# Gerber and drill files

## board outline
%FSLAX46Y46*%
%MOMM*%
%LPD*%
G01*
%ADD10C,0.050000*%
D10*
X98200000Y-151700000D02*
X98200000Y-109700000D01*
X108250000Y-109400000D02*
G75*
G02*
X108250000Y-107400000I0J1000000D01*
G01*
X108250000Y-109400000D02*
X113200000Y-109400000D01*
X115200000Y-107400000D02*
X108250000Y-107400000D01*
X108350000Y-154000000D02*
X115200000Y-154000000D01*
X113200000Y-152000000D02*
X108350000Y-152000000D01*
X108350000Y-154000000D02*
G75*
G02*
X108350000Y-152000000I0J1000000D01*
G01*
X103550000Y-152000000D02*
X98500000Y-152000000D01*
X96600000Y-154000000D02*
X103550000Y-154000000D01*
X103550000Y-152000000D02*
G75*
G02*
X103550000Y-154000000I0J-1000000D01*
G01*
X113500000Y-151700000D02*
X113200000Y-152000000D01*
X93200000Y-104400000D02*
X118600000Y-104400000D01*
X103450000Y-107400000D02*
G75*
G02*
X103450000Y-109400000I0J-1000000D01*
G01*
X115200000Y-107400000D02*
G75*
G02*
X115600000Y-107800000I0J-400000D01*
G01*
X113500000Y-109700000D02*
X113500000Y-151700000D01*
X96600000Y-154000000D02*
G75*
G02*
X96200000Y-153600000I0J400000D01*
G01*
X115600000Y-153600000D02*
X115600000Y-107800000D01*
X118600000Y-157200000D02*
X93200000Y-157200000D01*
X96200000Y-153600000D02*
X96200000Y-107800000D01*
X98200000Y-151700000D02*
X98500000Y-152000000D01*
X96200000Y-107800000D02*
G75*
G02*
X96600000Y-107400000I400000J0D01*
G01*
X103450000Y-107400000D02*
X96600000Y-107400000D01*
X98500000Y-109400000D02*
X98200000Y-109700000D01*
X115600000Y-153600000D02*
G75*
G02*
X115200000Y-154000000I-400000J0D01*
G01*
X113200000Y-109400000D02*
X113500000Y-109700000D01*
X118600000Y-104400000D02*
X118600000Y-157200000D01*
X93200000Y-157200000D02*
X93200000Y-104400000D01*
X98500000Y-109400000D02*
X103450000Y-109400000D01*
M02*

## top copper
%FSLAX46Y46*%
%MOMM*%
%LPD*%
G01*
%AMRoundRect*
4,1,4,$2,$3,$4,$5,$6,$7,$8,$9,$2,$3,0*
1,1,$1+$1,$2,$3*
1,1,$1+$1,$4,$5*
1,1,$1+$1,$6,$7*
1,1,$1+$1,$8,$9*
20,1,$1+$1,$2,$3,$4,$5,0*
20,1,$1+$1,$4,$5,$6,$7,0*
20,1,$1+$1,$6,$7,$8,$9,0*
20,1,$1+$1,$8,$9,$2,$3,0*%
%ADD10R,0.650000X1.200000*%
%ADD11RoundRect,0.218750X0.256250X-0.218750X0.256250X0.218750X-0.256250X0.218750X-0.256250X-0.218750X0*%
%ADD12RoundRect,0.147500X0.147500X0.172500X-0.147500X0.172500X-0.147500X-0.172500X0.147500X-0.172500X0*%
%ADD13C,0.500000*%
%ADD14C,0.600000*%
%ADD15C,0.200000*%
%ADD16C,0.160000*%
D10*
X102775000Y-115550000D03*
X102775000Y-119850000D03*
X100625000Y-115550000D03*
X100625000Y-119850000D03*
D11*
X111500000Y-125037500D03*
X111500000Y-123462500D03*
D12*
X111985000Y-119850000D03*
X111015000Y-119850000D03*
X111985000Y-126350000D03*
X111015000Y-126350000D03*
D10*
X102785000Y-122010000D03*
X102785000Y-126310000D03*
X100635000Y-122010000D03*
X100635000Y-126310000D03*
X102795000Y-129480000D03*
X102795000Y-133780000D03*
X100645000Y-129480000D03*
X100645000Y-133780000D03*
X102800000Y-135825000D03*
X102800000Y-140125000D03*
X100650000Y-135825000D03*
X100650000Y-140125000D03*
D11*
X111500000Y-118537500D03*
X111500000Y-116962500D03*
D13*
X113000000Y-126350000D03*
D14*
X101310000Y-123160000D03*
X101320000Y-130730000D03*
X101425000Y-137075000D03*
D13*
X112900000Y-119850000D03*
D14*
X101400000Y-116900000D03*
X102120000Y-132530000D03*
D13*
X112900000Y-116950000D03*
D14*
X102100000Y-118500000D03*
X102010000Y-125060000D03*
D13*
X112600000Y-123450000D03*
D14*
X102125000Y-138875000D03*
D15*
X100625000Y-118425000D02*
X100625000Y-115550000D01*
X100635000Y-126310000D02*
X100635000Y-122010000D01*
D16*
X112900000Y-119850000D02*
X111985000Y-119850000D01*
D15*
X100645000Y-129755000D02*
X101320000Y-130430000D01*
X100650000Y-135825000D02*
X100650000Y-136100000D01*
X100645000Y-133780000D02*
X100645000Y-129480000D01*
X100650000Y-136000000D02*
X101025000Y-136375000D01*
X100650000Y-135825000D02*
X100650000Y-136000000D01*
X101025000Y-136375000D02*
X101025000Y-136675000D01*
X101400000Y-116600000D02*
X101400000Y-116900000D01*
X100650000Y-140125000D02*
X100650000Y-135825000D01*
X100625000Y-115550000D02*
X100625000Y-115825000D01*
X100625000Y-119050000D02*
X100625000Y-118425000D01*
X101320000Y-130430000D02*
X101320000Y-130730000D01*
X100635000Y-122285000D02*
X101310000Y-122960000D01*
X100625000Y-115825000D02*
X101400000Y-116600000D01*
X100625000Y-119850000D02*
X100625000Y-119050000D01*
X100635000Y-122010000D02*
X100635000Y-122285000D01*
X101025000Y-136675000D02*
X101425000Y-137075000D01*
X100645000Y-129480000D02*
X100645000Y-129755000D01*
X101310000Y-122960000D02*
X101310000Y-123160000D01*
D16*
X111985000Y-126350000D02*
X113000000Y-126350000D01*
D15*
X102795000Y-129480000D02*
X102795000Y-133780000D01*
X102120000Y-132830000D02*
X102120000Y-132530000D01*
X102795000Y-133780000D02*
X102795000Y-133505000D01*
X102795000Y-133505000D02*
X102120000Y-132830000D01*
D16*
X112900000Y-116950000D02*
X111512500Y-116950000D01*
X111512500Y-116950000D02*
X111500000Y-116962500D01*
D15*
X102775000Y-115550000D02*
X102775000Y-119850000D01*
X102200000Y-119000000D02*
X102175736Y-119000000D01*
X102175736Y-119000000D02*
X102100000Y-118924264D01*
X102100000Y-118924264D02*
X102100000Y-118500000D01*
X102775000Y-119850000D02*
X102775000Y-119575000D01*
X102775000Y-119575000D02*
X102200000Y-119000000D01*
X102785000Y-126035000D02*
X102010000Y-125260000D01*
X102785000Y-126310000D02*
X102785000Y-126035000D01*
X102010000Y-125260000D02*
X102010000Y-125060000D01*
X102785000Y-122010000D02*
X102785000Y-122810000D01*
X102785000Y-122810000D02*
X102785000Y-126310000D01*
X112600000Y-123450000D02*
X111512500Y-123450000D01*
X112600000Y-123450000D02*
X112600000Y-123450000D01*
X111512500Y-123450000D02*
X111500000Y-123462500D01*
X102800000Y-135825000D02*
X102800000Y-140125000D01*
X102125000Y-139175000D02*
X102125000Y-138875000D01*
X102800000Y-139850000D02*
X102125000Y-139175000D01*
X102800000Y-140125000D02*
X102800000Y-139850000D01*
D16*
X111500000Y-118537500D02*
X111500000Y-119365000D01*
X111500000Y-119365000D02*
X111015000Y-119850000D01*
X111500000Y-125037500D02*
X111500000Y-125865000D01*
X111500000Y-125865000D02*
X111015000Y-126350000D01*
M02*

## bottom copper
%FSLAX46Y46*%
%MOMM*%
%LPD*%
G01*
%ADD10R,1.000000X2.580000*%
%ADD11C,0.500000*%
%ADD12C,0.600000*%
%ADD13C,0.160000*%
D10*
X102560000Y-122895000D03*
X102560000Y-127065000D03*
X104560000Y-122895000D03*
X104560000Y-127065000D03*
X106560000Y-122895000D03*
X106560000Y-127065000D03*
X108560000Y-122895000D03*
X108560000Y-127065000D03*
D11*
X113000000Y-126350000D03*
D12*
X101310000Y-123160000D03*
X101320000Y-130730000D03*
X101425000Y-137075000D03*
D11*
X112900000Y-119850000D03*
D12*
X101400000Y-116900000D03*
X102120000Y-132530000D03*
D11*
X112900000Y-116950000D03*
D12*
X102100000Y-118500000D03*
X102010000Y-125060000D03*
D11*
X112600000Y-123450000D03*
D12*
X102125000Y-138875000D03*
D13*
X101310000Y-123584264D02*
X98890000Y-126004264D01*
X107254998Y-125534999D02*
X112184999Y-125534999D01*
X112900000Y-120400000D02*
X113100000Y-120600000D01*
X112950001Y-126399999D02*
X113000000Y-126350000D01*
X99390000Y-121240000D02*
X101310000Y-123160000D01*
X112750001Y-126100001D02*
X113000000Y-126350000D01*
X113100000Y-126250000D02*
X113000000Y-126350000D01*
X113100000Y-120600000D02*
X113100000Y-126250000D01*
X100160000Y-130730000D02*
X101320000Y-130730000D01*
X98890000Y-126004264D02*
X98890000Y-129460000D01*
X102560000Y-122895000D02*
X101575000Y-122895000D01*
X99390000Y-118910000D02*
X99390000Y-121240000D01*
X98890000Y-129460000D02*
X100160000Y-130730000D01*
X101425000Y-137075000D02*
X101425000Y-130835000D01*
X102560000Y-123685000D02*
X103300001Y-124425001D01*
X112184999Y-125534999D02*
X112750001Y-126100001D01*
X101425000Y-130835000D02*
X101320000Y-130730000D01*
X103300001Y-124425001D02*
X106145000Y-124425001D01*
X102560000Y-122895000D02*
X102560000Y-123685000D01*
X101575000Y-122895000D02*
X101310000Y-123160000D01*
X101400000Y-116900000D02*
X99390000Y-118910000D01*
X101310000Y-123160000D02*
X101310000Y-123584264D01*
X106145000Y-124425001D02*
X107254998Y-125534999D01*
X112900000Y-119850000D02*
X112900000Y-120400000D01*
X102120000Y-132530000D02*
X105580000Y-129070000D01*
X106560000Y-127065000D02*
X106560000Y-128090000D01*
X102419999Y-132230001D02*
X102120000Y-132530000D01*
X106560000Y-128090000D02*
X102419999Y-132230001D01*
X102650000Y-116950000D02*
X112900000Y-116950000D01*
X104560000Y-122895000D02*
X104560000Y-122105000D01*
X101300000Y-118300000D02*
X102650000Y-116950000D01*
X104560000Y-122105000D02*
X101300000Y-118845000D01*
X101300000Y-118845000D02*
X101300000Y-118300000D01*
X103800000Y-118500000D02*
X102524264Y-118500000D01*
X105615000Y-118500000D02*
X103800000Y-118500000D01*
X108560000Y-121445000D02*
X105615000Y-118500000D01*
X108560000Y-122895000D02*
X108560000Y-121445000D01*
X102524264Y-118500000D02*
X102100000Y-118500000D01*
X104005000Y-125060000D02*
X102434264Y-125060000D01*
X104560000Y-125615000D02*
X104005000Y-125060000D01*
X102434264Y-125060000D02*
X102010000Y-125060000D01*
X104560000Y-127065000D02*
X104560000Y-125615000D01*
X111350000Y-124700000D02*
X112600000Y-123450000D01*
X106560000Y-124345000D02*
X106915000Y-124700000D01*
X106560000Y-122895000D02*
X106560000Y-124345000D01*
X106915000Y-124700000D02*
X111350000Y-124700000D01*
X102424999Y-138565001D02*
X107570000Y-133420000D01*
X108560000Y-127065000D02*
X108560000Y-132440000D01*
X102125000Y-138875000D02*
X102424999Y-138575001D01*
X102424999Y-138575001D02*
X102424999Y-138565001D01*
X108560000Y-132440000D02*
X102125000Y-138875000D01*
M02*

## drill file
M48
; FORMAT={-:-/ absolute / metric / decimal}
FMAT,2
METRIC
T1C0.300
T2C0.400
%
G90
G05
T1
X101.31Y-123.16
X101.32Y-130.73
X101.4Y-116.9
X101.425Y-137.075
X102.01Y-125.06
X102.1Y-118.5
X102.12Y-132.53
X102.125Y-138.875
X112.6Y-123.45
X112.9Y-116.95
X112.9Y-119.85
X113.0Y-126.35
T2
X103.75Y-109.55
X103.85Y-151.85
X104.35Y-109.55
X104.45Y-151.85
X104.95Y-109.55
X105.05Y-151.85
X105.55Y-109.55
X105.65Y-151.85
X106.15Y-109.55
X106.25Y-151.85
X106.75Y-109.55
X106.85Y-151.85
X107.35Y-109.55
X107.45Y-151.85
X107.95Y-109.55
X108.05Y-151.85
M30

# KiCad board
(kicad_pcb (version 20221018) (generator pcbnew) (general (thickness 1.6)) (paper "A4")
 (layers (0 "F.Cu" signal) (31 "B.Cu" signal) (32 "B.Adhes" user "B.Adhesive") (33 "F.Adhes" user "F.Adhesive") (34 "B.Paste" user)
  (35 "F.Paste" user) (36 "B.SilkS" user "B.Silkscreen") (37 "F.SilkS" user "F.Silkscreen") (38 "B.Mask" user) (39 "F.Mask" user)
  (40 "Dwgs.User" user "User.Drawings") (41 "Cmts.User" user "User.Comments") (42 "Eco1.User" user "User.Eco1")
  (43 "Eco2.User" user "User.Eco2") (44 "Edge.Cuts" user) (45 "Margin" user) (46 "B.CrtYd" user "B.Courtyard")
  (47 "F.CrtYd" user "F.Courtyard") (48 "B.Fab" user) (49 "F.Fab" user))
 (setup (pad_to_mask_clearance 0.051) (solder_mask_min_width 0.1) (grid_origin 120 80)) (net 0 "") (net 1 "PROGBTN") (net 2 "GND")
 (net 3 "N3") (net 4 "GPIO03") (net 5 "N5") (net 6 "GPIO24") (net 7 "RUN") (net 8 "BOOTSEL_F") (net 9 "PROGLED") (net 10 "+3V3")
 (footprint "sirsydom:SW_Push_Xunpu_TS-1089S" (layer "F.Cu") (at 101.7 117.7 -90)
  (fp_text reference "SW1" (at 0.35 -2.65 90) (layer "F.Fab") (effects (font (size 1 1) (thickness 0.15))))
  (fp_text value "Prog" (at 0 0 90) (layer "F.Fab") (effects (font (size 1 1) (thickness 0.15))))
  (pad "1" smd rect (at -2.15 -1.075 270) (size 1.2 0.65) (layers "F.Cu" "F.Paste" "F.Mask") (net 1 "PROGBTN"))
  (pad "1" smd rect (at 2.15 -1.075 270) (size 1.2 0.65) (layers "F.Cu" "F.Paste" "F.Mask") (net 1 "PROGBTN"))
  (pad "2" smd rect (at -2.15 1.075 270) (size 1.2 0.65) (layers "F.Cu" "F.Paste" "F.Mask") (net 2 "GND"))
  (pad "2" smd rect (at 2.15 1.075 270) (size 1.2 0.65) (layers "F.Cu" "F.Paste" "F.Mask") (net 2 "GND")))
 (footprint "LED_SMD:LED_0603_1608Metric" (layer "F.Cu") (at 111.5 124.25 90)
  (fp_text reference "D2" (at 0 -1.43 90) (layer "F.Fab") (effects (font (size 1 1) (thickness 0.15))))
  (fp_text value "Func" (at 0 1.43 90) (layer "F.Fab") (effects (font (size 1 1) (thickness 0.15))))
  (pad "1" smd roundrect (at -0.7875 0 90) (size 0.875 0.95) (layers "F.Cu" "F.Paste" "F.Mask") (roundrect_rratio 0.25) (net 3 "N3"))
  (pad "2" smd roundrect (at 0.7875 0 90) (size 0.875 0.95) (layers "F.Cu" "F.Paste" "F.Mask") (roundrect_rratio 0.25) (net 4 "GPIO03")))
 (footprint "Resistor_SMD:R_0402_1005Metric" (layer "F.Cu") (at 111.5 119.85 180)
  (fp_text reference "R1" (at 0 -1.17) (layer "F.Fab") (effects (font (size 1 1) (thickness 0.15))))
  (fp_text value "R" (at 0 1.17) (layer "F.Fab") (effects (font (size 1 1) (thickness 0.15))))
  (pad "1" smd roundrect (at -0.485 0 180) (size 0.59 0.64) (layers "F.Cu" "F.Paste" "F.Mask") (roundrect_rratio 0.25) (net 2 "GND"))
  (pad "2" smd roundrect (at 0.485 0 180) (size 0.59 0.64) (layers "F.Cu" "F.Paste" "F.Mask") (roundrect_rratio 0.25) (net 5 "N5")))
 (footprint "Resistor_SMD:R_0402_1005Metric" (layer "F.Cu") (at 111.5 126.35 180)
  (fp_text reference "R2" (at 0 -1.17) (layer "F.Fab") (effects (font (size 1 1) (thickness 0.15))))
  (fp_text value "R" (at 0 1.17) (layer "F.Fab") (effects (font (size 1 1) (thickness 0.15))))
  (pad "1" smd roundrect (at -0.485 0 180) (size 0.59 0.64) (layers "F.Cu" "F.Paste" "F.Mask") (roundrect_rratio 0.25) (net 2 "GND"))
  (pad "2" smd roundrect (at 0.485 0 180) (size 0.59 0.64) (layers "F.Cu" "F.Paste" "F.Mask") (roundrect_rratio 0.25) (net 3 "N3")))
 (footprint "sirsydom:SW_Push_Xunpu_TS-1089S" (layer "F.Cu") (at 101.71 124.16 -90)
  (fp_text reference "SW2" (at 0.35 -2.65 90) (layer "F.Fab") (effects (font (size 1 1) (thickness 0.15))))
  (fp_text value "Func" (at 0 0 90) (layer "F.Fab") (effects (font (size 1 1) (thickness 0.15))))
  (pad "1" smd rect (at -2.15 -1.075 270) (size 1.2 0.65) (layers "F.Cu" "F.Paste" "F.Mask") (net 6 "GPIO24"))
  (pad "1" smd rect (at 2.15 -1.075 270) (size 1.2 0.65) (layers "F.Cu" "F.Paste" "F.Mask") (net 6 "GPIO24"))
  (pad "2" smd rect (at -2.15 1.075 270) (size 1.2 0.65) (layers "F.Cu" "F.Paste" "F.Mask") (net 2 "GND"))
  (pad "2" smd rect (at 2.15 1.075 270) (size 1.2 0.65) (layers "F.Cu" "F.Paste" "F.Mask") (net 2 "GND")))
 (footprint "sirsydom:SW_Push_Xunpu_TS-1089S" (layer "F.Cu") (at 101.72 131.63 -90)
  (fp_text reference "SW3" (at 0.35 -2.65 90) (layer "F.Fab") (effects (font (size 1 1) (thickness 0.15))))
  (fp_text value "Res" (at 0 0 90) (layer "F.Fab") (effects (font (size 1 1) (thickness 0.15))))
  (pad "1" smd rect (at -2.15 -1.075 270) (size 1.2 0.65) (layers "F.Cu" "F.Paste" "F.Mask") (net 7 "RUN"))
  (pad "1" smd rect (at 2.15 -1.075 270) (size 1.2 0.65) (layers "F.Cu" "F.Paste" "F.Mask") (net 7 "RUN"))
  (pad "2" smd rect (at -2.15 1.075 270) (size 1.2 0.65) (layers "F.Cu" "F.Paste" "F.Mask") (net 2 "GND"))
  (pad "2" smd rect (at 2.15 1.075 270) (size 1.2 0.65) (layers "F.Cu" "F.Paste" "F.Mask") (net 2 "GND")))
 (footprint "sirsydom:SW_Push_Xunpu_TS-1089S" (layer "F.Cu") (at 101.725 137.975 -90)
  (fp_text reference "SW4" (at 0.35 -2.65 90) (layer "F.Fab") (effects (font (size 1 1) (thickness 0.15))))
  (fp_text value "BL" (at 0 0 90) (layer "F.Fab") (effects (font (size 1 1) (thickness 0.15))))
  (pad "1" smd rect (at -2.15 -1.075 270) (size 1.2 0.65) (layers "F.Cu" "F.Paste" "F.Mask") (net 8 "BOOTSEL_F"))
  (pad "1" smd rect (at 2.15 -1.075 270) (size 1.2 0.65) (layers "F.Cu" "F.Paste" "F.Mask") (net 8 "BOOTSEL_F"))
  (pad "2" smd rect (at -2.15 1.075 270) (size 1.2 0.65) (layers "F.Cu" "F.Paste" "F.Mask") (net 2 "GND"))
  (pad "2" smd rect (at 2.15 1.075 270) (size 1.2 0.65) (layers "F.Cu" "F.Paste" "F.Mask") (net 2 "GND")))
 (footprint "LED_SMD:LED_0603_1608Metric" (layer "F.Cu") (at 111.5 117.75 90)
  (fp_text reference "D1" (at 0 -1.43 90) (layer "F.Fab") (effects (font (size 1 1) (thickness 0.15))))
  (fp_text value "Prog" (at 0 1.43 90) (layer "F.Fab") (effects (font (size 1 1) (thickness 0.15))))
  (pad "1" smd roundrect (at -0.7875 0 90) (size 0.875 0.95) (layers "F.Cu" "F.Paste" "F.Mask") (roundrect_rratio 0.25) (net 5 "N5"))
  (pad "2" smd roundrect (at 0.7875 0 90) (size 0.875 0.95) (layers "F.Cu" "F.Paste" "F.Mask") (roundrect_rratio 0.25) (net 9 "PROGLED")))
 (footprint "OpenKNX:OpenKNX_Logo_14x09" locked (layer "F.Cu") (at 105.8 146.4)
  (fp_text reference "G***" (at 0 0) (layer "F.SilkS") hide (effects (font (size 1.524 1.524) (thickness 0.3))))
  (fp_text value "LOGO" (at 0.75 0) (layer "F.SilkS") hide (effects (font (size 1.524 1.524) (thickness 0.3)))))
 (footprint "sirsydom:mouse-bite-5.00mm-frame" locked (layer "F.Cu") (at 105.35 109.55)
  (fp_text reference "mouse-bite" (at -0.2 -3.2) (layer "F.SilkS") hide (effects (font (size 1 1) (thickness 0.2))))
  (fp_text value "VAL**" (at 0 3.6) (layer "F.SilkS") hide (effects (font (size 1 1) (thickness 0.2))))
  (pad "" np_thru_hole circle locked (at -1.6 0) (size 0.4 0.4) (drill 0.4) (layers "*.Cu" "*.Mask"))
  (pad "" np_thru_hole circle locked (at -1 0) (size 0.4 0.4) (drill 0.4) (layers "*.Cu" "*.Mask"))
  (pad "" np_thru_hole circle locked (at -0.4 0) (size 0.4 0.4) (drill 0.4) (layers "*.Cu" "*.Mask"))
  (pad "" np_thru_hole circle locked (at 0.2 0) (size 0.4 0.4) (drill 0.4) (layers "*.Cu" "*.Mask"))
  (pad "" np_thru_hole circle locked (at 0.8 0) (size 0.4 0.4) (drill 0.4) (layers "*.Cu" "*.Mask"))
  (pad "" np_thru_hole circle locked (at 1.4 0) (size 0.4 0.4) (drill 0.4) (layers "*.Cu" "*.Mask"))
  (pad "" np_thru_hole circle locked (at 2 0) (size 0.4 0.4) (drill 0.4) (layers "*.Cu" "*.Mask"))
  (pad "" np_thru_hole circle locked (at 2.6 0) (size 0.4 0.4) (drill 0.4) (layers "*.Cu" "*.Mask")))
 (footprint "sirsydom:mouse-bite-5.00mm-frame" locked (layer "F.Cu") (at 106.45 151.85 180)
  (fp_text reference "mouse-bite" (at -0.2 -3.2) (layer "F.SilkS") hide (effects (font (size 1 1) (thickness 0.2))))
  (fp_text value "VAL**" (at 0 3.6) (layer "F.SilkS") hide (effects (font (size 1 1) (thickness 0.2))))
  (pad "" np_thru_hole circle locked (at -1.6 0 180) (size 0.4 0.4) (drill 0.4) (layers "*.Cu" "*.Mask"))
  (pad "" np_thru_hole circle locked (at -1 0 180) (size 0.4 0.4) (drill 0.4) (layers "*.Cu" "*.Mask"))
  (pad "" np_thru_hole circle locked (at -0.4 0 180) (size 0.4 0.4) (drill 0.4) (layers "*.Cu" "*.Mask"))
  (pad "" np_thru_hole circle locked (at 0.2 0 180) (size 0.4 0.4) (drill 0.4) (layers "*.Cu" "*.Mask"))
  (pad "" np_thru_hole circle locked (at 0.8 0 180) (size 0.4 0.4) (drill 0.4) (layers "*.Cu" "*.Mask"))
  (pad "" np_thru_hole circle locked (at 1.4 0 180) (size 0.4 0.4) (drill 0.4) (layers "*.Cu" "*.Mask"))
  (pad "" np_thru_hole circle locked (at 2 0 180) (size 0.4 0.4) (drill 0.4) (layers "*.Cu" "*.Mask"))
  (pad "" np_thru_hole circle locked (at 2.6 0 180) (size 0.4 0.4) (drill 0.4) (layers "*.Cu" "*.Mask")))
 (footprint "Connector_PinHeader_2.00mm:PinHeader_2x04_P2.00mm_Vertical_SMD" (layer "B.Cu") (at 105.56 124.98 -90)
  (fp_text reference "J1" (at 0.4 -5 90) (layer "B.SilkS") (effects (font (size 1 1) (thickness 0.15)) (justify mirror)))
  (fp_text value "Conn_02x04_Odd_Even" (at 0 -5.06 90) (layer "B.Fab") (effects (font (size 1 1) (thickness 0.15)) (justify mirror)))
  (pad "1" smd rect (at -2.085 3 270) (size 2.58 1) (layers "B.Cu" "B.Paste" "B.Mask") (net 2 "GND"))
  (pad "2" smd rect (at 2.085 3 270) (size 2.58 1) (layers "B.Cu" "B.Paste" "B.Mask") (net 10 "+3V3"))
  (pad "3" smd rect (at -2.085 1 270) (size 2.58 1) (layers "B.Cu" "B.Paste" "B.Mask") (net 9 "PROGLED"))
  (pad "4" smd rect (at 2.085 1 270) (size 2.58 1) (layers "B.Cu" "B.Paste" "B.Mask") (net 6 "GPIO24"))
  (pad "5" smd rect (at -2.085 -1 270) (size 2.58 1) (layers "B.Cu" "B.Paste" "B.Mask") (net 4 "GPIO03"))
  (pad "6" smd rect (at 2.085 -1 270) (size 2.58 1) (layers "B.Cu" "B.Paste" "B.Mask") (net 7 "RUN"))
  (pad "7" smd rect (at -2.085 -3 270) (size 2.58 1) (layers "B.Cu" "B.Paste" "B.Mask") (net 1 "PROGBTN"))
  (pad "8" smd rect (at 2.085 -3 270) (size 2.58 1) (layers "B.Cu" "B.Paste" "B.Mask") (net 8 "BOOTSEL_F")))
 (gr_line (start 98.2 151.7) (end 98.2 109.7) (stroke (width 0.05) (type solid)) (layer "Edge.Cuts"))
 (gr_arc (start 108.25 109.4) (mid 107.25 108.4) (end 108.25 107.4) (stroke (width 0.05) (type solid)) (layer "Edge.Cuts"))
 (gr_line (start 108.25 109.4) (end 113.2 109.4) (stroke (width 0.05) (type solid)) (layer "Edge.Cuts"))
 (gr_line (start 115.2 107.4) (end 108.25 107.4) (stroke (width 0.05) (type solid)) (layer "Edge.Cuts"))
 (gr_line (start 108.35 154) (end 115.2 154) (stroke (width 0.05) (type solid)) (layer "Edge.Cuts"))
 (gr_line (start 113.2 152) (end 108.35 152) (stroke (width 0.05) (type solid)) (layer "Edge.Cuts"))
 (gr_arc (start 108.35 154) (mid 107.35 153) (end 108.35 152) (stroke (width 0.05) (type solid)) (layer "Edge.Cuts"))
 (gr_line (start 103.55 152) (end 98.5 152) (stroke (width 0.05) (type solid)) (layer "Edge.Cuts"))
 (gr_line (start 96.6 154) (end 103.55 154) (stroke (width 0.05) (type solid)) (layer "Edge.Cuts"))
 (gr_arc (start 103.55 152) (mid 104.55 153) (end 103.55 154) (stroke (width 0.05) (type solid)) (layer "Edge.Cuts"))
 (gr_line (start 113.5 151.7) (end 113.2 152) (stroke (width 0.05) (type solid)) (layer "Edge.Cuts"))
 (gr_line (start 93.2 104.4) (end 118.6 104.4) (stroke (width 0.05) (type solid)) (layer "Edge.Cuts"))
 (gr_arc (start 103.45 107.4) (mid 104.45 108.4) (end 103.45 109.4) (stroke (width 0.05) (type solid)) (layer "Edge.Cuts"))
 (gr_arc (start 115.2 107.4) (mid 115.482843 107.517157) (end 115.6 107.8) (stroke (width 0.05) (type solid)) (layer "Edge.Cuts"))
 (gr_line (start 113.5 109.7) (end 113.5 151.7) (stroke (width 0.05) (type solid)) (layer "Edge.Cuts"))
 (gr_arc (start 96.6 154) (mid 96.317157 153.882843) (end 96.2 153.6) (stroke (width 0.05) (type solid)) (layer "Edge.Cuts"))
 (gr_line (start 115.6 153.6) (end 115.6 107.8) (stroke (width 0.05) (type solid)) (layer "Edge.Cuts"))
 (gr_line (start 118.6 157.2) (end 93.2 157.2) (stroke (width 0.05) (type solid)) (layer "Edge.Cuts"))
 (gr_line (start 96.2 153.6) (end 96.2 107.8) (stroke (width 0.05) (type solid)) (layer "Edge.Cuts"))
 (gr_line (start 98.2 151.7) (end 98.5 152) (stroke (width 0.05) (type solid)) (layer "Edge.Cuts"))
 (gr_arc (start 96.2 107.8) (mid 96.317157 107.517157) (end 96.6 107.4) (stroke (width 0.05) (type solid)) (layer "Edge.Cuts"))
 (gr_line (start 103.45 107.4) (end 96.6 107.4) (stroke (width 0.05) (type solid)) (layer "Edge.Cuts"))
 (gr_line (start 98.5 109.4) (end 98.2 109.7) (stroke (width 0.05) (type solid)) (layer "Edge.Cuts"))
 (gr_arc (start 115.6 153.6) (mid 115.482843 153.882843) (end 115.2 154) (stroke (width 0.05) (type solid)) (layer "Edge.Cuts"))
 (gr_line (start 113.2 109.4) (end 113.5 109.7) (stroke (width 0.05) (type solid)) (layer "Edge.Cuts"))
 (gr_line (start 118.6 104.4) (end 118.6 157.2) (stroke (width 0.05) (type solid)) (layer "Edge.Cuts"))
 (gr_line (start 93.2 157.2) (end 93.2 104.4) (stroke (width 0.05) (type solid)) (layer "Edge.Cuts"))
 (gr_line (start 98.5 109.4) (end 103.45 109.4) (stroke (width 0.05) (type solid)) (layer "Edge.Cuts"))
 (segment (start 100.625 118.425) (end 100.625 115.55) (width 0.2) (layer "F.Cu") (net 2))
 (segment (start 100.635 126.31) (end 100.635 122.01) (width 0.2) (layer "F.Cu") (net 2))
 (segment (start 112.9 119.85) (end 111.985 119.85) (width 0.16) (layer "F.Cu") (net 2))
 (segment (start 100.645 129.755) (end 101.32 130.43) (width 0.2) (layer "F.Cu") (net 2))
 (segment (start 100.65 135.825) (end 100.65 136.1) (width 0.2) (layer "F.Cu") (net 2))
 (segment (start 100.645 133.78) (end 100.645 129.48) (width 0.2) (layer "F.Cu") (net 2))
 (segment (start 100.65 136) (end 101.025 136.375) (width 0.2) (layer "F.Cu") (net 2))
 (segment (start 100.65 135.825) (end 100.65 136) (width 0.2) (layer "F.Cu") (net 2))
 (segment (start 101.025 136.375) (end 101.025 136.675) (width 0.2) (layer "F.Cu") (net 2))
 (segment (start 101.4 116.6) (end 101.4 116.9) (width 0.2) (layer "F.Cu") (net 2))
 (segment (start 100.65 140.125) (end 100.65 135.825) (width 0.2) (layer "F.Cu") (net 2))
 (segment (start 100.625 115.55) (end 100.625 115.825) (width 0.2) (layer "F.Cu") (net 2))
 (segment (start 100.625 119.05) (end 100.625 118.425) (width 0.2) (layer "F.Cu") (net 2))
 (segment (start 101.32 130.43) (end 101.32 130.73) (width 0.2) (layer "F.Cu") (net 2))
 (segment (start 100.635 122.285) (end 101.31 122.96) (width 0.2) (layer "F.Cu") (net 2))
 (segment (start 100.625 115.825) (end 101.4 116.6) (width 0.2) (layer "F.Cu") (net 2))
 (segment (start 100.625 119.85) (end 100.625 119.05) (width 0.2) (layer "F.Cu") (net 2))
 (segment (start 100.635 122.01) (end 100.635 122.285) (width 0.2) (layer "F.Cu") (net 2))
 (segment (start 101.025 136.675) (end 101.425 137.075) (width 0.2) (layer "F.Cu") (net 2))
 (segment (start 100.645 129.48) (end 100.645 129.755) (width 0.2) (layer "F.Cu") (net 2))
 (segment (start 101.31 122.96) (end 101.31 123.16) (width 0.2) (layer "F.Cu") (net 2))
 (segment (start 111.985 126.35) (end 113 126.35) (width 0.16) (layer "F.Cu") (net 2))
 (via (at 113 126.35) (size 0.5) (drill 0.3) (layers "F.Cu" "B.Cu") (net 2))
 (via (at 101.31 123.16) (size 0.6) (drill 0.3) (layers "F.Cu" "B.Cu") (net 2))
 (via (at 101.32 130.73) (size 0.6) (drill 0.3) (layers "F.Cu" "B.Cu") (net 2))
 (via (at 101.425 137.075) (size 0.6) (drill 0.3) (layers "F.Cu" "B.Cu") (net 2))
 (via (at 112.9 119.85) (size 0.5) (drill 0.3) (layers "F.Cu" "B.Cu") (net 2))
 (via (at 101.4 116.9) (size 0.6) (drill 0.3) (layers "F.Cu" "B.Cu") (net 2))
 (segment (start 101.31 123.584264) (end 98.89 126.004264) (width 0.16) (layer "B.Cu") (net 2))
 (segment (start 107.254998 125.534999) (end 112.184999 125.534999) (width 0.16) (layer "B.Cu") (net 2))
 (segment (start 112.9 120.4) (end 113.1 120.6) (width 0.16) (layer "B.Cu") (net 2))
 (segment (start 112.950001 126.399999) (end 113 126.35) (width 0.16) (layer "B.Cu") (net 2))
 (segment (start 99.39 121.24) (end 101.31 123.16) (width 0.16) (layer "B.Cu") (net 2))
 (segment (start 112.750001 126.100001) (end 113 126.35) (width 0.16) (layer "B.Cu") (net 2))
 (segment (start 113.1 126.25) (end 113 126.35) (width 0.16) (layer "B.Cu") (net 2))
 (segment (start 113.1 120.6) (end 113.1 126.25) (width 0.16) (layer "B.Cu") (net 2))
 (segment (start 100.16 130.73) (end 101.32 130.73) (width 0.16) (layer "B.Cu") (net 2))
 (segment (start 98.89 126.004264) (end 98.89 129.46) (width 0.16) (layer "B.Cu") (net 2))
 (segment (start 102.56 122.895) (end 101.575 122.895) (width 0.16) (layer "B.Cu") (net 2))
 (segment (start 99.39 118.91) (end 99.39 121.24) (width 0.16) (layer "B.Cu") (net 2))
 (segment (start 98.89 129.46) (end 100.16 130.73) (width 0.16) (layer "B.Cu") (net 2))
 (segment (start 101.425 137.075) (end 101.425 130.835) (width 0.16) (layer "B.Cu") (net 2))
 (segment (start 102.56 123.685) (end 103.300001 124.425001) (width 0.16) (layer "B.Cu") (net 2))
 (segment (start 112.184999 125.534999) (end 112.750001 126.100001) (width 0.16) (layer "B.Cu") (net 2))
 (segment (start 101.425 130.835) (end 101.32 130.73) (width 0.16) (layer "B.Cu") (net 2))
 (segment (start 103.300001 124.425001) (end 106.145 124.425001) (width 0.16) (layer "B.Cu") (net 2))
 (segment (start 102.56 122.895) (end 102.56 123.685) (width 0.16) (layer "B.Cu") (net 2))
 (segment (start 101.575 122.895) (end 101.31 123.16) (width 0.16) (layer "B.Cu") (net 2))
 (segment (start 101.4 116.9) (end 99.39 118.91) (width 0.16) (layer "B.Cu") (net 2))
 (segment (start 101.31 123.16) (end 101.31 123.584264) (width 0.16) (layer "B.Cu") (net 2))
 (segment (start 106.145 124.425001) (end 107.254998 125.534999) (width 0.16) (layer "B.Cu") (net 2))
 (segment (start 112.9 119.85) (end 112.9 120.4) (width 0.16) (layer "B.Cu") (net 2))
 (segment (start 102.795 129.48) (end 102.795 133.78) (width 0.2) (layer "F.Cu") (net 7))
 (segment (start 102.12 132.83) (end 102.12 132.53) (width 0.2) (layer "F.Cu") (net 7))
 (segment (start 102.795 133.78) (end 102.795 133.505) (width 0.2) (layer "F.Cu") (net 7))
 (segment (start 102.795 133.505) (end 102.12 132.83) (width 0.2) (layer "F.Cu") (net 7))
 (via (at 102.12 132.53) (size 0.6) (drill 0.3) (layers "F.Cu" "B.Cu") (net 7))
 (segment (start 102.12 132.53) (end 105.58 129.07) (width 0.16) (layer "B.Cu") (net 7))
 (segment (start 106.56 127.065) (end 106.56 128.09) (width 0.16) (layer "B.Cu") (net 7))
 (segment (start 102.419999 132.230001) (end 102.12 132.53) (width 0.16) (layer "B.Cu") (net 7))
 (segment (start 106.56 128.09) (end 102.419999 132.230001) (width 0.16) (layer "B.Cu") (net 7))
 (segment (start 112.9 116.95) (end 111.5125 116.95) (width 0.16) (layer "F.Cu") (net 9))
 (segment (start 111.5125 116.95) (end 111.5 116.9625) (width 0.16) (layer "F.Cu") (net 9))
 (via (at 112.9 116.95) (size 0.5) (drill 0.3) (layers "F.Cu" "B.Cu") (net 9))
 (segment (start 102.65 116.95) (end 112.9 116.95) (width 0.16) (layer "B.Cu") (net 9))
 (segment (start 104.56 122.895) (end 104.56 122.105) (width 0.16) (layer "B.Cu") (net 9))
 (segment (start 101.3 118.3) (end 102.65 116.95) (width 0.16) (layer "B.Cu") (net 9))
 (segment (start 104.56 122.105) (end 101.3 118.845) (width 0.16) (layer "B.Cu") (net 9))
 (segment (start 101.3 118.845) (end 101.3 118.3) (width 0.16) (layer "B.Cu") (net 9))
 (segment (start 102.775 115.55) (end 102.775 119.85) (width 0.2) (layer "F.Cu") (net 1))
 (segment (start 102.2 119) (end 102.175736 119) (width 0.2) (layer "F.Cu") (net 1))
 (segment (start 102.175736 119) (end 102.1 118.924264) (width 0.2) (layer "F.Cu") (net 1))
 (segment (start 102.1 118.924264) (end 102.1 118.5) (width 0.2) (layer "F.Cu") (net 1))
 (segment (start 102.775 119.85) (end 102.775 119.575) (width 0.2) (layer "F.Cu") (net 1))
 (segment (start 102.775 119.575) (end 102.2 119) (width 0.2) (layer "F.Cu") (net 1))
 (via (at 102.1 118.5) (size 0.6) (drill 0.3) (layers "F.Cu" "B.Cu") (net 1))
 (segment (start 103.8 118.5) (end 102.524264 118.5) (width 0.16) (layer "B.Cu") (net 1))
 (segment (start 105.615 118.5) (end 103.8 118.5) (width 0.16) (layer "B.Cu") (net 1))
 (segment (start 108.56 121.445) (end 105.615 118.5) (width 0.16) (layer "B.Cu") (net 1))
 (segment (start 108.56 122.895) (end 108.56 121.445) (width 0.16) (layer "B.Cu") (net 1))
 (segment (start 102.524264 118.5) (end 102.1 118.5) (width 0.16) (layer "B.Cu") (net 1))
 (segment (start 102.785 126.035) (end 102.01 125.26) (width 0.2) (layer "F.Cu") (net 6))
 (segment (start 102.785 126.31) (end 102.785 126.035) (width 0.2) (layer "F.Cu") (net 6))
 (segment (start 102.01 125.26) (end 102.01 125.06) (width 0.2) (layer "F.Cu") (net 6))
 (segment (start 102.785 122.01) (end 102.785 122.81) (width 0.2) (layer "F.Cu") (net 6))
 (segment (start 102.785 122.81) (end 102.785 126.31) (width 0.2) (layer "F.Cu") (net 6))
 (via (at 102.01 125.06) (size 0.6) (drill 0.3) (layers "F.Cu" "B.Cu") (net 6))
 (segment (start 104.005 125.06) (end 102.434264 125.06) (width 0.16) (layer "B.Cu") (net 6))
 (segment (start 104.56 125.615) (end 104.005 125.06) (width 0.16) (layer "B.Cu") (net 6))
 (segment (start 102.434264 125.06) (end 102.01 125.06) (width 0.16) (layer "B.Cu") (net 6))
 (segment (start 104.56 127.065) (end 104.56 125.615) (width 0.16) (layer "B.Cu") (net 6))
 (segment (start 112.6 123.45) (end 111.5125 123.45) (width 0.2) (layer "F.Cu") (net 4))
 (segment (start 112.6 123.45) (end 112.6 123.45) (width 0.2) (layer "F.Cu") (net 4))
 (segment (start 111.5125 123.45) (end 111.5 123.4625) (width 0.2) (layer "F.Cu") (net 4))
 (via (at 112.6 123.45) (size 0.5) (drill 0.3) (layers "F.Cu" "B.Cu") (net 4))
 (segment (start 111.35 124.7) (end 112.6 123.45) (width 0.16) (layer "B.Cu") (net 4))
 (segment (start 106.56 124.345) (end 106.915 124.7) (width 0.16) (layer "B.Cu") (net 4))
 (segment (start 106.56 122.895) (end 106.56 124.345) (width 0.16) (layer "B.Cu") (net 4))
 (segment (start 106.915 124.7) (end 111.35 124.7) (width 0.16) (layer "B.Cu") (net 4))
 (segment (start 102.8 135.825) (end 102.8 140.125) (width 0.2) (layer "F.Cu") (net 8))
 (segment (start 102.125 139.175) (end 102.125 138.875) (width 0.2) (layer "F.Cu") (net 8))
 (segment (start 102.8 139.85) (end 102.125 139.175) (width 0.2) (layer "F.Cu") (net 8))
 (segment (start 102.8 140.125) (end 102.8 139.85) (width 0.2) (layer "F.Cu") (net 8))
 (via (at 102.125 138.875) (size 0.6) (drill 0.3) (layers "F.Cu" "B.Cu") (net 8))
 (segment (start 102.424999 138.565001) (end 107.57 133.42) (width 0.16) (layer "B.Cu") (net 8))
 (segment (start 108.56 127.065) (end 108.56 132.44) (width 0.16) (layer "B.Cu") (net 8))
 (segment (start 102.125 138.875) (end 102.424999 138.575001) (width 0.16) (layer "B.Cu") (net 8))
 (segment (start 102.424999 138.575001) (end 102.424999 138.565001) (width 0.16) (layer "B.Cu") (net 8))
 (segment (start 108.56 132.44) (end 102.125 138.875) (width 0.16) (layer "B.Cu") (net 8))
 (segment (start 111.5 118.5375) (end 111.5 119.365) (width 0.16) (layer "F.Cu") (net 5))
 (segment (start 111.5 119.365) (end 111.015 119.85) (width 0.16) (layer "F.Cu") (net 5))
 (segment (start 111.5 125.0375) (end 111.5 125.865) (width 0.16) (layer "F.Cu") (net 3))
 (segment (start 111.5 125.865) (end 111.015 126.35) (width 0.16) (layer "F.Cu") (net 3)))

